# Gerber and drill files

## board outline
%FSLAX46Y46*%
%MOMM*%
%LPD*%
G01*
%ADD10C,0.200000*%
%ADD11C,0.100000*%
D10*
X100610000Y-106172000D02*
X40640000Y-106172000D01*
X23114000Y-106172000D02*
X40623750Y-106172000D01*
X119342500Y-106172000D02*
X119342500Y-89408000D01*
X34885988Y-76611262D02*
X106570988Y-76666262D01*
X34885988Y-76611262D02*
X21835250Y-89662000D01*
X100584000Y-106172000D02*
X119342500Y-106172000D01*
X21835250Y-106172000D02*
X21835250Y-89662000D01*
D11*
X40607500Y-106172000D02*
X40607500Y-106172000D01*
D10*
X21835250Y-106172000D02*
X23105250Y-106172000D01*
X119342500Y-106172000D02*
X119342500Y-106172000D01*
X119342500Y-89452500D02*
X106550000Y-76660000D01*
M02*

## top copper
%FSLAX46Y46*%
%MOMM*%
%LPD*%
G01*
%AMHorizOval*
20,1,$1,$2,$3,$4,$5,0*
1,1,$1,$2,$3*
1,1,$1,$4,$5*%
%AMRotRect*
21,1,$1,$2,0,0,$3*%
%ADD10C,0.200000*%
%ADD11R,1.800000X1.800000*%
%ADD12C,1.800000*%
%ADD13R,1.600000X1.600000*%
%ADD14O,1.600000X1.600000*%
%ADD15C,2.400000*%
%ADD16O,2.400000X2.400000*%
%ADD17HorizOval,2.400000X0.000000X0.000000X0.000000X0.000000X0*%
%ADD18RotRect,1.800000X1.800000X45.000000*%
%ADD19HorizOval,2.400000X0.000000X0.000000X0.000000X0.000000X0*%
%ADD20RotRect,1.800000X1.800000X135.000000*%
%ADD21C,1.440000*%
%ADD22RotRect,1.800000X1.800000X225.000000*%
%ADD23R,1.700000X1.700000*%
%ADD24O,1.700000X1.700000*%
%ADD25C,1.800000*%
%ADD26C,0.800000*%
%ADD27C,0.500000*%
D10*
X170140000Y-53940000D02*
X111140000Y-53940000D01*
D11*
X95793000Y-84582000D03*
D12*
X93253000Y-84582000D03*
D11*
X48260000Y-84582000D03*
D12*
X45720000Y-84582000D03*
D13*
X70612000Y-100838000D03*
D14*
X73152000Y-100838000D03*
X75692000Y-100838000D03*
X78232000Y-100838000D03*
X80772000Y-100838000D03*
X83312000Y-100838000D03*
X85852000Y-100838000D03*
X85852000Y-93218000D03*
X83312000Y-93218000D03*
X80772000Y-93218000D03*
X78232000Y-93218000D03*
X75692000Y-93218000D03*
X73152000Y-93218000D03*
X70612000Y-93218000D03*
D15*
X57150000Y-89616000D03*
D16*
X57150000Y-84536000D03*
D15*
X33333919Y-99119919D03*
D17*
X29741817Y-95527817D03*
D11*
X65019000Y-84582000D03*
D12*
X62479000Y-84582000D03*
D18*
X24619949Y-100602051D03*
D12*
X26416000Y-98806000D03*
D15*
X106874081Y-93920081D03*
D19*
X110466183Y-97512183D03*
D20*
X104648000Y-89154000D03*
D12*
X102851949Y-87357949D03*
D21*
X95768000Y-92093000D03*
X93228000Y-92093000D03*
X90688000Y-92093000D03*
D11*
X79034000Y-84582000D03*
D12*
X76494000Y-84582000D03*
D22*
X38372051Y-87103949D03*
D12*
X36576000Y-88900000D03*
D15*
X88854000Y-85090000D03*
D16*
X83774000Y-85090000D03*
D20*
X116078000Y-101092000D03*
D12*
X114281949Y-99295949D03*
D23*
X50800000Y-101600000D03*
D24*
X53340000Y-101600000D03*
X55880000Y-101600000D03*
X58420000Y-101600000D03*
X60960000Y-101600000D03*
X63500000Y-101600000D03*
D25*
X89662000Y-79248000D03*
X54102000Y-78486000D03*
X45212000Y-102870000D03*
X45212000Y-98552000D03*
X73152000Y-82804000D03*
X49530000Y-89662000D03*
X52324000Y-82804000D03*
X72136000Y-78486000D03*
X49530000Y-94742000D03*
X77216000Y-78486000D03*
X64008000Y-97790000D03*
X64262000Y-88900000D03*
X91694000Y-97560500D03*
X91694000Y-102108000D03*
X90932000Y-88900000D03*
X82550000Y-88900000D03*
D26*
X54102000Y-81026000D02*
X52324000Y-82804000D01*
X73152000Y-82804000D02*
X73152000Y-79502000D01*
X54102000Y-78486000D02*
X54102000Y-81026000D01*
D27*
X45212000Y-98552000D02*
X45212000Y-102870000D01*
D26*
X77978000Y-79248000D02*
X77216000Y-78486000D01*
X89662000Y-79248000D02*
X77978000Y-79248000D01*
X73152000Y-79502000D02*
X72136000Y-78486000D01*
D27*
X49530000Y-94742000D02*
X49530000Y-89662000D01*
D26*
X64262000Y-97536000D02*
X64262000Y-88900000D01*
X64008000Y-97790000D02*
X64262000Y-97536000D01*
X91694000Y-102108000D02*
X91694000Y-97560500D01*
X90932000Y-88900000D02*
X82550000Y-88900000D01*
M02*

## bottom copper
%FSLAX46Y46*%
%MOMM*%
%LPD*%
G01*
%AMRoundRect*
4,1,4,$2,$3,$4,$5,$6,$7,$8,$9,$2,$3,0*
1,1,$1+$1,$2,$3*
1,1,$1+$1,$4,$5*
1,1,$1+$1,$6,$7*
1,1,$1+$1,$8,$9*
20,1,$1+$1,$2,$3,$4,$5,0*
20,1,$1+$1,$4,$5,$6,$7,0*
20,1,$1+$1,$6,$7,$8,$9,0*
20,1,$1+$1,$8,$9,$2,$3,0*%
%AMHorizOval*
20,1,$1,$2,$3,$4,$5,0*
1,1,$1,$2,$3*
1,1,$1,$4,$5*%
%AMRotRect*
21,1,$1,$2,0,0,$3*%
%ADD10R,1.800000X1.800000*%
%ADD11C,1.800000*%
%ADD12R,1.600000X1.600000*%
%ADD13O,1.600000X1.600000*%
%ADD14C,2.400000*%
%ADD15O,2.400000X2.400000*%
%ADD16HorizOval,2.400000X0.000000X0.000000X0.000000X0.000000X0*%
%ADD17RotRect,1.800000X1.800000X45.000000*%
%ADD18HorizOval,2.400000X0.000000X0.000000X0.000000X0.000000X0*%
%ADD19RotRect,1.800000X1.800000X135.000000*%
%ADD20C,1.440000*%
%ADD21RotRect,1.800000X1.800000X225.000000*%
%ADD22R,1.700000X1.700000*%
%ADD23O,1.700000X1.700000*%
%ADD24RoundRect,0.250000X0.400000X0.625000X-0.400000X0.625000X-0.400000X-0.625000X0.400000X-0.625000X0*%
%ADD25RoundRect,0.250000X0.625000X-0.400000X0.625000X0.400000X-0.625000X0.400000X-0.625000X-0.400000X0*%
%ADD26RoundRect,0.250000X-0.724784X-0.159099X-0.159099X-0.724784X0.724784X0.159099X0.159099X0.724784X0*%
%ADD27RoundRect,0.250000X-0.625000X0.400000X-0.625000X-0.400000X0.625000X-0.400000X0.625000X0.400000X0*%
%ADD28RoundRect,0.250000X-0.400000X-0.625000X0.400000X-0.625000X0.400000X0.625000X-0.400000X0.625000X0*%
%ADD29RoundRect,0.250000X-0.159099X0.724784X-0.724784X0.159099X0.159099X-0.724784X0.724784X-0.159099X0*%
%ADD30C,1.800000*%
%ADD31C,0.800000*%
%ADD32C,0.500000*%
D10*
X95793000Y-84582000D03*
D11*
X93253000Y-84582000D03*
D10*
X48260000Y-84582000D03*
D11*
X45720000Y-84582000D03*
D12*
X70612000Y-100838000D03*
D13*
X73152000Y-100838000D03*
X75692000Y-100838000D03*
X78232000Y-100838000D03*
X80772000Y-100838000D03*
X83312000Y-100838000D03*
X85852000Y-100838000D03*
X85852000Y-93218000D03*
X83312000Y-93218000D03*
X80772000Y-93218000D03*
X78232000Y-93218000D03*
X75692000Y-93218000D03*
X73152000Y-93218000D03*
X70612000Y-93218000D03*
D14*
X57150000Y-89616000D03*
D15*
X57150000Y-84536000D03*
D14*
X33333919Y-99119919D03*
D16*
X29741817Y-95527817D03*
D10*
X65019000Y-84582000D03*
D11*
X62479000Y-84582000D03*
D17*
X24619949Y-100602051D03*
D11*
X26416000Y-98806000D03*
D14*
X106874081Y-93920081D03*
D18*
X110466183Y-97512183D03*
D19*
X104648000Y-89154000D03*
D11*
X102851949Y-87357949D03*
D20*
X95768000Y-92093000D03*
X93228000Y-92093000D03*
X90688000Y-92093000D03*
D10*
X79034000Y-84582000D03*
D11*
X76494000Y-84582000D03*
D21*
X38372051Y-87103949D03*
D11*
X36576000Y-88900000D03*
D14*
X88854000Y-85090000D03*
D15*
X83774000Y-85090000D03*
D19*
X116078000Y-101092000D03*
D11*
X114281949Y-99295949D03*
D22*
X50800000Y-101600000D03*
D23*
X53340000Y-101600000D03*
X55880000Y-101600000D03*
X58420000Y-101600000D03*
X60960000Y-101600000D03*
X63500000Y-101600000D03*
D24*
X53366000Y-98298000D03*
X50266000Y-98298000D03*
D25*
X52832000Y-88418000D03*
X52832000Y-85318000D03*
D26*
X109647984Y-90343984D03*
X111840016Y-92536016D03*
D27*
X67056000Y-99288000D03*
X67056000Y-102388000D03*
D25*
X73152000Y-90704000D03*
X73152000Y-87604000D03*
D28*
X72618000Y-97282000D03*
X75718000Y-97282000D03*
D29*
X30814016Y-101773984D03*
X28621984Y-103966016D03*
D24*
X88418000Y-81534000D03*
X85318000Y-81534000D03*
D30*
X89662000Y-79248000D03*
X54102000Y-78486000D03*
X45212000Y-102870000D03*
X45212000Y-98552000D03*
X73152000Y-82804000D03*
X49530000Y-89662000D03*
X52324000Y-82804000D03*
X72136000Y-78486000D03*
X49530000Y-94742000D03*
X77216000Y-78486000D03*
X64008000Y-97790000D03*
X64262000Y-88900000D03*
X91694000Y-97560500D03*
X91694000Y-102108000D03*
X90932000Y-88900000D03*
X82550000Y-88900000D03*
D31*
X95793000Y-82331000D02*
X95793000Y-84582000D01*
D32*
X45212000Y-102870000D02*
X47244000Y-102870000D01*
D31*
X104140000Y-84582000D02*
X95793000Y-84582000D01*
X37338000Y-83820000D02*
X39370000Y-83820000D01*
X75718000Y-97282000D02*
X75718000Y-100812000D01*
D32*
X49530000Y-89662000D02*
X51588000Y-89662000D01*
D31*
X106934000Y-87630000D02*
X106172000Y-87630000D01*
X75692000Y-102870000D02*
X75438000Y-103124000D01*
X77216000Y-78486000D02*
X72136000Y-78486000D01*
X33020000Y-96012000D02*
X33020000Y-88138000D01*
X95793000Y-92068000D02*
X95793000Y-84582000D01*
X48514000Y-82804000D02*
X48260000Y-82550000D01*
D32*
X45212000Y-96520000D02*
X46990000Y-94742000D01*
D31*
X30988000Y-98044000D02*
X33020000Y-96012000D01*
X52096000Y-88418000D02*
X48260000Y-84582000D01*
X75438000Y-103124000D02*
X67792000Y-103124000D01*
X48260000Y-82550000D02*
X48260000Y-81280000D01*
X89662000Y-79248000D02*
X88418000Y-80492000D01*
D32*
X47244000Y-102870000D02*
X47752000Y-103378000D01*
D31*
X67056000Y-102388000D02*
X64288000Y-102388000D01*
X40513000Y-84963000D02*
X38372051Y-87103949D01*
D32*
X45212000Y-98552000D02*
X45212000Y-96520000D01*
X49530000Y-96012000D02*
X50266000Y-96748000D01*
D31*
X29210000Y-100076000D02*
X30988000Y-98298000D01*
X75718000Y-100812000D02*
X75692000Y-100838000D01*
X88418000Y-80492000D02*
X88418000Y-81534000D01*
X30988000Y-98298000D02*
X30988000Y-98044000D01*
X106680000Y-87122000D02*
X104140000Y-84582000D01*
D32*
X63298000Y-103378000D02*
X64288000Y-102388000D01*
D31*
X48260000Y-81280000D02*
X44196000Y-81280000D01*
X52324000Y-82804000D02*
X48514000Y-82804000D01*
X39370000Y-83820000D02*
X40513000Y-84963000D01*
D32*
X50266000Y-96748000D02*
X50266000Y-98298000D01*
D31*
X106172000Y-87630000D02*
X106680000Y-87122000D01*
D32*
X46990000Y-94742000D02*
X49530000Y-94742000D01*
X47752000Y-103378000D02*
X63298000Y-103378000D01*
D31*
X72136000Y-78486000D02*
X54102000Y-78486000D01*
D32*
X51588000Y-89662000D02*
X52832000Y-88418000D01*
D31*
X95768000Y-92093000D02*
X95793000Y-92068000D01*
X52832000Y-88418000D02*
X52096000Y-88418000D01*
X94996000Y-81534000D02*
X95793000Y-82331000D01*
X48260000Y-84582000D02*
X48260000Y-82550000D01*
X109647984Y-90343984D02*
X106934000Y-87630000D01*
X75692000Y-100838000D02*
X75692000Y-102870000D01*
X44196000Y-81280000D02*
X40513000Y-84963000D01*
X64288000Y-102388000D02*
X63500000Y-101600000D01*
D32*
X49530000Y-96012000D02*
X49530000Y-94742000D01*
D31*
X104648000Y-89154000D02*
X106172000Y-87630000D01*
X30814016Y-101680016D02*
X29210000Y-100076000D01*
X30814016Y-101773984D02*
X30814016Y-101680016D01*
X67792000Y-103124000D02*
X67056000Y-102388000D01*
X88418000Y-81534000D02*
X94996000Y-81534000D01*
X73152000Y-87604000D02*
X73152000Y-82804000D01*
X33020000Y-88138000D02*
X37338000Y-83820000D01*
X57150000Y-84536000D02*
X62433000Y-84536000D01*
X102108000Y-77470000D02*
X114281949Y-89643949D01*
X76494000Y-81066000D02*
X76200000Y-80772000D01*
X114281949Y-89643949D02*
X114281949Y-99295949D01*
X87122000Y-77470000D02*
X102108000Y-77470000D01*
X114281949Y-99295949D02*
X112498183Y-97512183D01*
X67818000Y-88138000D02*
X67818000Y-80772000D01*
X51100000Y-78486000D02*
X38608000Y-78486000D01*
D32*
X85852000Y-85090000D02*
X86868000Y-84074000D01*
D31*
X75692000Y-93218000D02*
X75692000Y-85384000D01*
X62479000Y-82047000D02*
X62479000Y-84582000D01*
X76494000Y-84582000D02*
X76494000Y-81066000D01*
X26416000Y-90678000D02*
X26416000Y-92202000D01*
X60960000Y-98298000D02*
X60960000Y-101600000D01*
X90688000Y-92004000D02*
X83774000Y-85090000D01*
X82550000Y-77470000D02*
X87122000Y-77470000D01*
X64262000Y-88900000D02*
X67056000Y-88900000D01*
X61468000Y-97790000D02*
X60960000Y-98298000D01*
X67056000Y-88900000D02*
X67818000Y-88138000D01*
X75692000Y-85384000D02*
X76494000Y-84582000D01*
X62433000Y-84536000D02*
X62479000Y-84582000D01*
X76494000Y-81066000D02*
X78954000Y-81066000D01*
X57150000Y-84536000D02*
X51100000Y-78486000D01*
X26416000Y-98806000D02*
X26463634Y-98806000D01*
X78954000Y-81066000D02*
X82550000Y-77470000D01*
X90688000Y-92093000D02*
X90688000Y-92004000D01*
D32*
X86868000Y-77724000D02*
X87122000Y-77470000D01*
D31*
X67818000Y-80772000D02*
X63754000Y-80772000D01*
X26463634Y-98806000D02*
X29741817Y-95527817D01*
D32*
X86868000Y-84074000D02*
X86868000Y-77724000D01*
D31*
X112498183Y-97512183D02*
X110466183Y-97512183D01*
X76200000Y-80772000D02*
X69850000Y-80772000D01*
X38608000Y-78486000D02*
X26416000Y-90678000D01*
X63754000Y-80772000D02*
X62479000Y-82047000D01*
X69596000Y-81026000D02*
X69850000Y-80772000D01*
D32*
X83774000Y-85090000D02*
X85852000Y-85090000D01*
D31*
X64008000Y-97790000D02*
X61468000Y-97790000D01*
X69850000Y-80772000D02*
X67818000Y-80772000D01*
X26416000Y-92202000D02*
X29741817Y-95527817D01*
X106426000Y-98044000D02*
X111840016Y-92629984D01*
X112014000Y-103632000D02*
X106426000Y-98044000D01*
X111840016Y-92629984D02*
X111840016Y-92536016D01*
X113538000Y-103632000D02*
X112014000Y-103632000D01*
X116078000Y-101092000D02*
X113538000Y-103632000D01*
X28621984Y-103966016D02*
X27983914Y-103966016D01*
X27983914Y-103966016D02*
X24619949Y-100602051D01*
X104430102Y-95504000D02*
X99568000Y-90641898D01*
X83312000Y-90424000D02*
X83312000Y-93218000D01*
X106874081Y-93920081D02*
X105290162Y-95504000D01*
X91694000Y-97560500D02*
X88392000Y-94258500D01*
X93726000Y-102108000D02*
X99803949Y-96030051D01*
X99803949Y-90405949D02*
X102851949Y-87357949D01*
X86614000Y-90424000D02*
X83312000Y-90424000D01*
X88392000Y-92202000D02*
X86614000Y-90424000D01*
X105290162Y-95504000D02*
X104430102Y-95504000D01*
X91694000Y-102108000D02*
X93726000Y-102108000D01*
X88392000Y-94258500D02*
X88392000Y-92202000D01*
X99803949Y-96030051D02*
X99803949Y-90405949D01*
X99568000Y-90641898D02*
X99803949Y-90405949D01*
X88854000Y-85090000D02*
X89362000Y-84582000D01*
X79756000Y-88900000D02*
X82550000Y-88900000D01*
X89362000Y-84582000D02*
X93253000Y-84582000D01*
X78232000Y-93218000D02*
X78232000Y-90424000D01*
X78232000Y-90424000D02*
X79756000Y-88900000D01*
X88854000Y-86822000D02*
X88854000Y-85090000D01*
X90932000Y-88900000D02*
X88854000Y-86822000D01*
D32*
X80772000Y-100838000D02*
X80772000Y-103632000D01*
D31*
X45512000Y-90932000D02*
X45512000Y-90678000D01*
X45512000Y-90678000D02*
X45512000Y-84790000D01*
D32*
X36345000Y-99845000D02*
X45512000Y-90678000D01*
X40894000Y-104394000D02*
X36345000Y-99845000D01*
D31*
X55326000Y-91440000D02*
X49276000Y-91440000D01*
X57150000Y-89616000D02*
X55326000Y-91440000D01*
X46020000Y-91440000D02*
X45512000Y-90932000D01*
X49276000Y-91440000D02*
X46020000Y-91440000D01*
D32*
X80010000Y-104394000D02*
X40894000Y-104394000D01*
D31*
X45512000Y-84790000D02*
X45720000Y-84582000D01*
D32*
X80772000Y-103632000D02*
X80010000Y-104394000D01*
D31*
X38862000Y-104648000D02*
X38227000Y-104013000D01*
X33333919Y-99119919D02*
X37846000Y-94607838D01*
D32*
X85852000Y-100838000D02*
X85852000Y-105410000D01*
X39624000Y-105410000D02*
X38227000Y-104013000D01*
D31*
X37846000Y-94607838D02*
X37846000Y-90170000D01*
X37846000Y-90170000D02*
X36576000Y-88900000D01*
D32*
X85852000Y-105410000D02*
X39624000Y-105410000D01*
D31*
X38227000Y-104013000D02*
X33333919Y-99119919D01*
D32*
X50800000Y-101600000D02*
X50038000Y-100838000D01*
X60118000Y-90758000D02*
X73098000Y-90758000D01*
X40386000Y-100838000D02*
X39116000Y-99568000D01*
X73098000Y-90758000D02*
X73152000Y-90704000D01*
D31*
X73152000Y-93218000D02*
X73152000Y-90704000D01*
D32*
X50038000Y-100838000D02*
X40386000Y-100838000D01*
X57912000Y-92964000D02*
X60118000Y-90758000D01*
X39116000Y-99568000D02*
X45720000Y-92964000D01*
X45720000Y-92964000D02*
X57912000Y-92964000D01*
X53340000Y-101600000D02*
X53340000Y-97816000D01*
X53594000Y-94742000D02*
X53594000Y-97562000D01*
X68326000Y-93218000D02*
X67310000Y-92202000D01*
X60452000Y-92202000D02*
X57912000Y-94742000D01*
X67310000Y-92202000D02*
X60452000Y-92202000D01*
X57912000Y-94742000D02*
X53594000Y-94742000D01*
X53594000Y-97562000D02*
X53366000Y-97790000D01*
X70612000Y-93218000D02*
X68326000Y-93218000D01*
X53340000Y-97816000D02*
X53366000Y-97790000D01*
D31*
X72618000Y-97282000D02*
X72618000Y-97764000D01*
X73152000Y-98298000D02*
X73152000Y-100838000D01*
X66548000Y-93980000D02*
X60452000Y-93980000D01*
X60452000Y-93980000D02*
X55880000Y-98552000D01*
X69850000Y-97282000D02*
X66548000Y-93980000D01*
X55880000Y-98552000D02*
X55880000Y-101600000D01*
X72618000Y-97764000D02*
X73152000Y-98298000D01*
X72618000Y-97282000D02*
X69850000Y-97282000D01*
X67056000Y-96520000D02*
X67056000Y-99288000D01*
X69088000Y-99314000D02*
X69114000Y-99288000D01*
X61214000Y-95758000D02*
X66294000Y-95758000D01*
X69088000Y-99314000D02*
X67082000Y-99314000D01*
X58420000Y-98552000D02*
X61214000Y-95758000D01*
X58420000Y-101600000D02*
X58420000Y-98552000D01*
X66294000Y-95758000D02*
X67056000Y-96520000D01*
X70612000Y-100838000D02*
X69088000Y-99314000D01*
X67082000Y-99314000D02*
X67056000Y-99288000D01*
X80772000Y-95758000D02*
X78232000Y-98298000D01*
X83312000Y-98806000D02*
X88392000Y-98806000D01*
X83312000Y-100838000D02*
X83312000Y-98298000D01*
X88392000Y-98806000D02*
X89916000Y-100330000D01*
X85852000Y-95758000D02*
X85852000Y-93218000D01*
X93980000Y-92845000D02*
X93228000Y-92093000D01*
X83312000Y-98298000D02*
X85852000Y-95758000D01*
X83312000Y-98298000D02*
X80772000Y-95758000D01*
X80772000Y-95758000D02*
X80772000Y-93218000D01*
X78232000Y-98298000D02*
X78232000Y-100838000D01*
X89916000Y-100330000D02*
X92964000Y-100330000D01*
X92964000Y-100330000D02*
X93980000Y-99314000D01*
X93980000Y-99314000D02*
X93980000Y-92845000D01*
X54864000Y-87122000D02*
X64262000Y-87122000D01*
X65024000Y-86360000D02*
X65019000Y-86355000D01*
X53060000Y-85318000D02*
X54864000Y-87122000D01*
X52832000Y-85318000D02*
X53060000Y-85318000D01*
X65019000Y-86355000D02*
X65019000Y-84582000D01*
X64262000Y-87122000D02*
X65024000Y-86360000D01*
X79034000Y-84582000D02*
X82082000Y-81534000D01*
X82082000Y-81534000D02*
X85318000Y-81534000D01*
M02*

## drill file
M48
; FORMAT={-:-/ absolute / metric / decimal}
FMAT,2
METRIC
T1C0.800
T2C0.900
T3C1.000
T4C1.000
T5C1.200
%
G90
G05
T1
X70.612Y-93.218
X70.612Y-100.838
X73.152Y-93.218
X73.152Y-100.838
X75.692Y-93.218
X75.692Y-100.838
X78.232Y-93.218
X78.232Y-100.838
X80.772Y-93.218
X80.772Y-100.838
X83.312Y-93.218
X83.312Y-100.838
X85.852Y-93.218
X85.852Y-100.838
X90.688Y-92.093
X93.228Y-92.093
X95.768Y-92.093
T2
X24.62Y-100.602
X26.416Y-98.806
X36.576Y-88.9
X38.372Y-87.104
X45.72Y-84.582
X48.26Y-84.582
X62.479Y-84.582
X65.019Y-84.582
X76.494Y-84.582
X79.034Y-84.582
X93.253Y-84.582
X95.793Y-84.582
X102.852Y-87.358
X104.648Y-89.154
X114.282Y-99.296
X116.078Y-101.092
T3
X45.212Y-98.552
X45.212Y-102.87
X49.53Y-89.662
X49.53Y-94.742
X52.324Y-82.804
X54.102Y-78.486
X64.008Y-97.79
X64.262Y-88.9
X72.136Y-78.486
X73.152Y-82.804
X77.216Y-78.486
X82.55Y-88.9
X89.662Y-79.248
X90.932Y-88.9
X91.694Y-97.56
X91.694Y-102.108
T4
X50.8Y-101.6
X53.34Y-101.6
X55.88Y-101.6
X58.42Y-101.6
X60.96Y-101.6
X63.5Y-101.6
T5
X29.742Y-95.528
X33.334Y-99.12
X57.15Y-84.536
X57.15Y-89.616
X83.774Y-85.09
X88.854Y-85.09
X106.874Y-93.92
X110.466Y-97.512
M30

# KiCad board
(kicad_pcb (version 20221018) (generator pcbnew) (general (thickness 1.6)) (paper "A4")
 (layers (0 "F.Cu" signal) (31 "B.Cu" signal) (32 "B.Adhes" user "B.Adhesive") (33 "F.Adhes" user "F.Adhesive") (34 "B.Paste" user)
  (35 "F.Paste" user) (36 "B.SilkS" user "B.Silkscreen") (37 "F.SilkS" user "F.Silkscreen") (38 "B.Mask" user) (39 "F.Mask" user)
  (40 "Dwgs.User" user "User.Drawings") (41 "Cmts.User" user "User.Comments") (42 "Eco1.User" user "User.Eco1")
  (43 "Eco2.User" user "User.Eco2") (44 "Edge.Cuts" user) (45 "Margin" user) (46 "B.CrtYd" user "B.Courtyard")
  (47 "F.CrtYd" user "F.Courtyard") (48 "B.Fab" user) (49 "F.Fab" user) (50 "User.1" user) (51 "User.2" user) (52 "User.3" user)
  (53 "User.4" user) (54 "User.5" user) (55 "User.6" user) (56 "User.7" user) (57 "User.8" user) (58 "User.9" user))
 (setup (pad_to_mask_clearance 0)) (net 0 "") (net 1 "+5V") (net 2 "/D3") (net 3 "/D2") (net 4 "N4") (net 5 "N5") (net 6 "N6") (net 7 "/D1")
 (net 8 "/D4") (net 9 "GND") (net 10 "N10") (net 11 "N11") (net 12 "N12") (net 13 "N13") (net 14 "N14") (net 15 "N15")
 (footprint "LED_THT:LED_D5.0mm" (layer "F.Cu") (at 95.793 84.582 180)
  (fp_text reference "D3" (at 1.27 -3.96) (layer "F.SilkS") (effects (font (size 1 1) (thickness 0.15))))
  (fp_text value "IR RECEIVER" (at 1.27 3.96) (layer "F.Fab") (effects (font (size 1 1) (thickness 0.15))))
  (pad "1" thru_hole rect (at 0 0 180) (size 1.8 1.8) (drill 0.9) (layers "*.Cu" "*.Mask") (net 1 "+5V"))
  (pad "2" thru_hole circle (at 2.54 0 180) (size 1.8 1.8) (drill 0.9) (layers "*.Cu" "*.Mask") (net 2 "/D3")))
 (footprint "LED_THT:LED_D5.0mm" (layer "F.Cu") (at 48.26 84.582 180)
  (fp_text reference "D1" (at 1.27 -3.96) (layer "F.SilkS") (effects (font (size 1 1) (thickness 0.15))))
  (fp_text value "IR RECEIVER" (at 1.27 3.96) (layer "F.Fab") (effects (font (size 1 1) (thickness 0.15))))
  (pad "1" thru_hole rect (at 0 0 180) (size 1.8 1.8) (drill 0.9) (layers "*.Cu" "*.Mask") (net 1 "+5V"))
  (pad "2" thru_hole circle (at 2.54 0 180) (size 1.8 1.8) (drill 0.9) (layers "*.Cu" "*.Mask") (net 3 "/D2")))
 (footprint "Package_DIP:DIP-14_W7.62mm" (layer "F.Cu") (at 70.612 100.838 90)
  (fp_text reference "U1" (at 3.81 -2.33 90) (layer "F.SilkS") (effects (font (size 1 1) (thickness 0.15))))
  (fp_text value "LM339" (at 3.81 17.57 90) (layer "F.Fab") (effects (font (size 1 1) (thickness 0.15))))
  (pad "1" thru_hole rect (at 0 0 90) (size 1.6 1.6) (drill 0.8) (layers "*.Cu" "*.Mask") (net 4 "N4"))
  (pad "2" thru_hole oval (at 0 2.54 90) (size 1.6 1.6) (drill 0.8) (layers "*.Cu" "*.Mask") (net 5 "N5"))
  (pad "3" thru_hole oval (at 0 5.08 90) (size 1.6 1.6) (drill 0.8) (layers "*.Cu" "*.Mask") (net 1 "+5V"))
  (pad "4" thru_hole oval (at 0 7.62 90) (size 1.6 1.6) (drill 0.8) (layers "*.Cu" "*.Mask") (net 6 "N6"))
  (pad "5" thru_hole oval (at 0 10.16 90) (size 1.6 1.6) (drill 0.8) (layers "*.Cu" "*.Mask") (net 3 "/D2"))
  (pad "6" thru_hole oval (at 0 12.7 90) (size 1.6 1.6) (drill 0.8) (layers "*.Cu" "*.Mask") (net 6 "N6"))
  (pad "7" thru_hole oval (at 0 15.24 90) (size 1.6 1.6) (drill 0.8) (layers "*.Cu" "*.Mask") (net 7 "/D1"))
  (pad "8" thru_hole oval (at 7.62 15.24 90) (size 1.6 1.6) (drill 0.8) (layers "*.Cu" "*.Mask") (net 6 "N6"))
  (pad "9" thru_hole oval (at 7.62 12.7 90) (size 1.6 1.6) (drill 0.8) (layers "*.Cu" "*.Mask") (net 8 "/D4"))
  (pad "10" thru_hole oval (at 7.62 10.16 90) (size 1.6 1.6) (drill 0.8) (layers "*.Cu" "*.Mask") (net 6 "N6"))
  (pad "11" thru_hole oval (at 7.62 7.62 90) (size 1.6 1.6) (drill 0.8) (layers "*.Cu" "*.Mask") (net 2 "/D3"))
  (pad "12" thru_hole oval (at 7.62 5.08 90) (size 1.6 1.6) (drill 0.8) (layers "*.Cu" "*.Mask") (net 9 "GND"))
  (pad "13" thru_hole oval (at 7.62 2.54 90) (size 1.6 1.6) (drill 0.8) (layers "*.Cu" "*.Mask") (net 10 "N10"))
  (pad "14" thru_hole oval (at 7.62 0 90) (size 1.6 1.6) (drill 0.8) (layers "*.Cu" "*.Mask") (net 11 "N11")))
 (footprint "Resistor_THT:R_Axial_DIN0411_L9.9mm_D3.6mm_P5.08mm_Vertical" (layer "F.Cu") (at 57.15 89.616 90)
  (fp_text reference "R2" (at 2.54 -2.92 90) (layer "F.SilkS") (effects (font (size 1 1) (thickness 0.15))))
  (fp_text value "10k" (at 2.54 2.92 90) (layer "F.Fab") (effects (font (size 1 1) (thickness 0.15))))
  (pad "1" thru_hole circle (at 0 0 90) (size 2.4 2.4) (drill 1.2) (layers "*.Cu" "*.Mask") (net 3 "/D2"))
  (pad "2" thru_hole oval (at 5.08 0 90) (size 2.4 2.4) (drill 1.2) (layers "*.Cu" "*.Mask") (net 9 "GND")))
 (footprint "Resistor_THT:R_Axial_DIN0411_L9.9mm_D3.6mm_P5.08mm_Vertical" (layer "F.Cu") (at 33.333919 99.119919 135)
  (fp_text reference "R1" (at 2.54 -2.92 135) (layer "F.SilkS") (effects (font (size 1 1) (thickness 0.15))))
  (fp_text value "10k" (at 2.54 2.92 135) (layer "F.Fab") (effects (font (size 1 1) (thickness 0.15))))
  (pad "1" thru_hole circle (at 0 0 135) (size 2.4 2.4) (drill 1.2) (layers "*.Cu" "*.Mask") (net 7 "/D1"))
  (pad "2" thru_hole oval (at 5.08 0 135) (size 2.4 2.4) (drill 1.2) (layers "*.Cu" "*.Mask") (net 9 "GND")))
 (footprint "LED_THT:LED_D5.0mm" (layer "F.Cu") (at 65.019 84.582 180)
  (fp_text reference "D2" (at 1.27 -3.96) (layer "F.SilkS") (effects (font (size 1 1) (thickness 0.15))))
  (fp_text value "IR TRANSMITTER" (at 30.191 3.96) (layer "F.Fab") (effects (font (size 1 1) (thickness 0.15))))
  (pad "1" thru_hole rect (at 0 0 180) (size 1.8 1.8) (drill 0.9) (layers "*.Cu" "*.Mask") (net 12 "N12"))
  (pad "2" thru_hole circle (at 2.54 0 180) (size 1.8 1.8) (drill 0.9) (layers "*.Cu" "*.Mask") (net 9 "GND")))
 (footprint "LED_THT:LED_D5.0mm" (layer "F.Cu") (at 24.619949 100.602051 45)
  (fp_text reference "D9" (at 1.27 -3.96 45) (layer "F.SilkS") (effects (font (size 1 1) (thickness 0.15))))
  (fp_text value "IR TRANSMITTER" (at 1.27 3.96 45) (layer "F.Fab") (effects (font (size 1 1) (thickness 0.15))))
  (pad "1" thru_hole rect (at 0 0 45) (size 1.8 1.8) (drill 0.9) (layers "*.Cu" "*.Mask") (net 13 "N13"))
  (pad "2" thru_hole circle (at 2.54 0 45) (size 1.8 1.8) (drill 0.9) (layers "*.Cu" "*.Mask") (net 9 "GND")))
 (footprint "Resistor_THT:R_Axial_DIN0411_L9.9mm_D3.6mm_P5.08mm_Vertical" (layer "F.Cu") (at 106.874081 93.920081 -45)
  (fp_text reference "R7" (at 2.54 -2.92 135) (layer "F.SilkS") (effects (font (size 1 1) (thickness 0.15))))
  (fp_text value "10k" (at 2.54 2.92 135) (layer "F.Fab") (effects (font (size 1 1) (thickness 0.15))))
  (pad "1" thru_hole circle (at 0 0 315) (size 2.4 2.4) (drill 1.2) (layers "*.Cu" "*.Mask") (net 8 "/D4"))
  (pad "2" thru_hole oval (at 5.08 0 315) (size 2.4 2.4) (drill 1.2) (layers "*.Cu" "*.Mask") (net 9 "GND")))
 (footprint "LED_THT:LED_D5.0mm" (layer "F.Cu") (at 104.648 89.154 135)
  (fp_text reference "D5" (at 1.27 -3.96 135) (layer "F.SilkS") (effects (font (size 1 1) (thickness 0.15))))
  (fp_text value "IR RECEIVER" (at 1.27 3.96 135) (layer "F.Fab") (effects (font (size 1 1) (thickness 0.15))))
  (pad "1" thru_hole rect (at 0 0 135) (size 1.8 1.8) (drill 0.9) (layers "*.Cu" "*.Mask") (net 1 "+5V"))
  (pad "2" thru_hole circle (at 2.54 0 135) (size 1.8 1.8) (drill 0.9) (layers "*.Cu" "*.Mask") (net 8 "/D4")))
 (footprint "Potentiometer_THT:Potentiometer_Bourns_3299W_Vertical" (layer "F.Cu") (at 95.768 92.093)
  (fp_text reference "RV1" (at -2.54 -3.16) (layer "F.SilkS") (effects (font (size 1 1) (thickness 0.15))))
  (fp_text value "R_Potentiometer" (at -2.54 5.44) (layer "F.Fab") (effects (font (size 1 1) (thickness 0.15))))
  (pad "1" thru_hole circle (at 0 0) (size 1.44 1.44) (drill 0.8) (layers "*.Cu" "*.Mask") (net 1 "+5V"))
  (pad "2" thru_hole circle (at -2.54 0) (size 1.44 1.44) (drill 0.8) (layers "*.Cu" "*.Mask") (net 6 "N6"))
  (pad "3" thru_hole circle (at -5.08 0) (size 1.44 1.44) (drill 0.8) (layers "*.Cu" "*.Mask") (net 9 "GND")))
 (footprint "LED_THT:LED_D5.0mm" (layer "F.Cu") (at 79.034 84.582 180)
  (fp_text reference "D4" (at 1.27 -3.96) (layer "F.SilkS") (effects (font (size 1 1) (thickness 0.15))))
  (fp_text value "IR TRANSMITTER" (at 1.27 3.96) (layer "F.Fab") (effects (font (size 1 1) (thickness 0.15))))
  (pad "1" thru_hole rect (at 0 0 180) (size 1.8 1.8) (drill 0.9) (layers "*.Cu" "*.Mask") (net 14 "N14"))
  (pad "2" thru_hole circle (at 2.54 0 180) (size 1.8 1.8) (drill 0.9) (layers "*.Cu" "*.Mask") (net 9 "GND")))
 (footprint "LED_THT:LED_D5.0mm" (layer "F.Cu") (at 38.372051 87.103949 -135)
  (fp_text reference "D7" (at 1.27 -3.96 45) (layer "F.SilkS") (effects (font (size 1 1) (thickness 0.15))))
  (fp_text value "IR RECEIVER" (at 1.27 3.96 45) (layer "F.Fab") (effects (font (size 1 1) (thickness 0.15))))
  (pad "1" thru_hole rect (at 0 0 225) (size 1.8 1.8) (drill 0.9) (layers "*.Cu" "*.Mask") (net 1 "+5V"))
  (pad "2" thru_hole circle (at 2.54 0 225) (size 1.8 1.8) (drill 0.9) (layers "*.Cu" "*.Mask") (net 7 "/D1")))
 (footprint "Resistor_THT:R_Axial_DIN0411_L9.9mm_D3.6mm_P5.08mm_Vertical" (layer "F.Cu") (at 88.854 85.09 180)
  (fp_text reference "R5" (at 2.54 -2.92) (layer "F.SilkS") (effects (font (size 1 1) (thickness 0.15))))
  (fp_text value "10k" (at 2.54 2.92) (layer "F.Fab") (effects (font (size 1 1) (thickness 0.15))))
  (pad "1" thru_hole circle (at 0 0 180) (size 2.4 2.4) (drill 1.2) (layers "*.Cu" "*.Mask") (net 2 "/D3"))
  (pad "2" thru_hole oval (at 5.08 0 180) (size 2.4 2.4) (drill 1.2) (layers "*.Cu" "*.Mask") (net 9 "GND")))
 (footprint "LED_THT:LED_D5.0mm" (layer "F.Cu") (at 116.078 101.092 135)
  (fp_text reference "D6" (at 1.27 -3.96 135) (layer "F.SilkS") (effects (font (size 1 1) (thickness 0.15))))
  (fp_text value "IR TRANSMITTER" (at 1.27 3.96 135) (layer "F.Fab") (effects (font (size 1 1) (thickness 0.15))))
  (pad "1" thru_hole rect (at 0 0 135) (size 1.8 1.8) (drill 0.9) (layers "*.Cu" "*.Mask") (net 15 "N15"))
  (pad "2" thru_hole circle (at 2.54 0 135) (size 1.8 1.8) (drill 0.9) (layers "*.Cu" "*.Mask") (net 9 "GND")))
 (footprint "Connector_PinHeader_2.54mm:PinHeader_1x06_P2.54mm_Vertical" (layer "F.Cu") (at 50.8 101.6 90)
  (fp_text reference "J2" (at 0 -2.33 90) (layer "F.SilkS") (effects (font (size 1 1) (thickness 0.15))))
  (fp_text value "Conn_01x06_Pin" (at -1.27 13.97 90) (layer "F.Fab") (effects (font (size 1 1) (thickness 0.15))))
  (pad "1" thru_hole rect (at 0 0 90) (size 1.7 1.7) (drill 1) (layers "*.Cu" "*.Mask") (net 10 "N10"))
  (pad "2" thru_hole oval (at 0 2.54 90) (size 1.7 1.7) (drill 1) (layers "*.Cu" "*.Mask") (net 11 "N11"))
  (pad "3" thru_hole oval (at 0 5.08 90) (size 1.7 1.7) (drill 1) (layers "*.Cu" "*.Mask") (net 5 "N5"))
  (pad "4" thru_hole oval (at 0 7.62 90) (size 1.7 1.7) (drill 1) (layers "*.Cu" "*.Mask") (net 4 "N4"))
  (pad "5" thru_hole oval (at 0 10.16 90) (size 1.7 1.7) (drill 1) (layers "*.Cu" "*.Mask") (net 9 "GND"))
  (pad "6" thru_hole oval (at 0 12.7 90) (size 1.7 1.7) (drill 1) (layers "*.Cu" "*.Mask") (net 1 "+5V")))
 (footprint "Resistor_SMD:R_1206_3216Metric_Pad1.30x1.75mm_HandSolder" (layer "B.Cu") (at 51.816 98.298 180)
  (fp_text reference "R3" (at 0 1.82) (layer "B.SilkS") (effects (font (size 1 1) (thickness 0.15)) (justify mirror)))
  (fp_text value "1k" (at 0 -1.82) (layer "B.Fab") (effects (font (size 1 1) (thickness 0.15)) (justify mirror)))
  (pad "1" smd roundrect (at -1.55 0 180) (size 1.3 1.75) (layers "B.Cu" "B.Paste" "B.Mask") (roundrect_rratio 0.192308) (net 11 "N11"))
  (pad "2" smd roundrect (at 1.55 0 180) (size 1.3 1.75) (layers "B.Cu" "B.Paste" "B.Mask") (roundrect_rratio 0.192308) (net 1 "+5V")))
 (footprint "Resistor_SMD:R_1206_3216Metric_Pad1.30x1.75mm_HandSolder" (layer "B.Cu") (at 52.832 86.868 90)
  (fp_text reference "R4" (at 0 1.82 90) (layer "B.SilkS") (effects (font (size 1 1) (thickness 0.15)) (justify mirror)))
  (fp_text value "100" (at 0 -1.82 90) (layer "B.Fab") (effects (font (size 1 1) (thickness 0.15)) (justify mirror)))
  (pad "1" smd roundrect (at -1.55 0 90) (size 1.3 1.75) (layers "B.Cu" "B.Paste" "B.Mask") (roundrect_rratio 0.192308) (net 1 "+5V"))
  (pad "2" smd roundrect (at 1.55 0 90) (size 1.3 1.75) (layers "B.Cu" "B.Paste" "B.Mask") (roundrect_rratio 0.192308) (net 12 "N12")))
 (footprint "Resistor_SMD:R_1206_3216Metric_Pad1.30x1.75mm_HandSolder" (layer "B.Cu") (at 110.744 91.44 -45)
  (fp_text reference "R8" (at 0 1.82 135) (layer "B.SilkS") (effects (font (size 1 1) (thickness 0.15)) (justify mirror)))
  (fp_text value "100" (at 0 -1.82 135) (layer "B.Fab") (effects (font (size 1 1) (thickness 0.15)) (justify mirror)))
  (pad "1" smd roundrect (at -1.55 0 315) (size 1.3 1.75) (layers "B.Cu" "B.Paste" "B.Mask") (roundrect_rratio 0.192308) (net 1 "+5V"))
  (pad "2" smd roundrect (at 1.55 0 315) (size 1.3 1.75) (layers "B.Cu" "B.Paste" "B.Mask") (roundrect_rratio 0.192308) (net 15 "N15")))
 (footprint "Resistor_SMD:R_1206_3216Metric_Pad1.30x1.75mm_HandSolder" (layer "B.Cu") (at 67.056 100.838 -90)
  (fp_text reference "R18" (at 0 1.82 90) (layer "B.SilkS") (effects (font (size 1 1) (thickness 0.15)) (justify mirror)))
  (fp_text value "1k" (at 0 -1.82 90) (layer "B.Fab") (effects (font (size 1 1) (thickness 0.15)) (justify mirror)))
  (pad "1" smd roundrect (at -1.55 0 270) (size 1.3 1.75) (layers "B.Cu" "B.Paste" "B.Mask") (roundrect_rratio 0.192308) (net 4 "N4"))
  (pad "2" smd roundrect (at 1.55 0 270) (size 1.3 1.75) (layers "B.Cu" "B.Paste" "B.Mask") (roundrect_rratio 0.192308) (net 1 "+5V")))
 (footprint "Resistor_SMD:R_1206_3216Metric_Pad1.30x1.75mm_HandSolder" (layer "B.Cu") (at 73.152 89.154 90)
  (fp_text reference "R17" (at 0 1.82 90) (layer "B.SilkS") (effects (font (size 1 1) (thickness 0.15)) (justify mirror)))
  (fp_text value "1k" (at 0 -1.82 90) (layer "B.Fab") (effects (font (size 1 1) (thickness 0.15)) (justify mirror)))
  (pad "1" smd roundrect (at -1.55 0 90) (size 1.3 1.75) (layers "B.Cu" "B.Paste" "B.Mask") (roundrect_rratio 0.192308) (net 10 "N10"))
  (pad "2" smd roundrect (at 1.55 0 90) (size 1.3 1.75) (layers "B.Cu" "B.Paste" "B.Mask") (roundrect_rratio 0.192308) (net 1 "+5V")))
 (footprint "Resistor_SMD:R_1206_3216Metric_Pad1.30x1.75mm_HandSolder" (layer "B.Cu") (at 74.168 97.282)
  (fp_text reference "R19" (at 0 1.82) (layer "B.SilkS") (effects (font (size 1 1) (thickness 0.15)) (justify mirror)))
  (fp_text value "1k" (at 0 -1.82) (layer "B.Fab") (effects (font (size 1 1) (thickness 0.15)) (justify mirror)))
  (pad "1" smd roundrect (at -1.55 0) (size 1.3 1.75) (layers "B.Cu" "B.Paste" "B.Mask") (roundrect_rratio 0.192308) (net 5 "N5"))
  (pad "2" smd roundrect (at 1.55 0) (size 1.3 1.75) (layers "B.Cu" "B.Paste" "B.Mask") (roundrect_rratio 0.192308) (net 1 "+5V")))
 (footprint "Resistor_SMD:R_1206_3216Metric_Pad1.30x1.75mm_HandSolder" (layer "B.Cu") (at 29.718 102.87 -135)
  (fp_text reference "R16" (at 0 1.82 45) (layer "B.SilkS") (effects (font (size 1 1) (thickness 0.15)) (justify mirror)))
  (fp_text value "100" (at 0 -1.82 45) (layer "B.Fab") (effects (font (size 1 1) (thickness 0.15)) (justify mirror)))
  (pad "1" smd roundrect (at -1.55 0 225) (size 1.3 1.75) (layers "B.Cu" "B.Paste" "B.Mask") (roundrect_rratio 0.192308) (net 1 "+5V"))
  (pad "2" smd roundrect (at 1.55 0 225) (size 1.3 1.75) (layers "B.Cu" "B.Paste" "B.Mask") (roundrect_rratio 0.192308) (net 13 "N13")))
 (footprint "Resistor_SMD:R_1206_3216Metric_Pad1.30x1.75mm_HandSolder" (layer "B.Cu") (at 86.868 81.534 180)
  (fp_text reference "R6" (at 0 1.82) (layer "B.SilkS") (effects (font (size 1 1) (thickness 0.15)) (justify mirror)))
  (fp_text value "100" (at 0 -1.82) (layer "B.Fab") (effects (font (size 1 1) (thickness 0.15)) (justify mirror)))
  (pad "1" smd roundrect (at -1.55 0 180) (size 1.3 1.75) (layers "B.Cu" "B.Paste" "B.Mask") (roundrect_rratio 0.192308) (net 1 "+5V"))
  (pad "2" smd roundrect (at 1.55 0 180) (size 1.3 1.75) (layers "B.Cu" "B.Paste" "B.Mask") (roundrect_rratio 0.192308) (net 14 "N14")))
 (gr_line locked (start 170.14 53.94) (end 111.14 53.94) (stroke (width 0.2) (type default)) (layer "F.Cu"))
 (gr_line (start 100.61 106.172) (end 40.64 106.172) (stroke (width 0.2) (type default)) (layer "Edge.Cuts"))
 (gr_line (start 23.114 106.172) (end 40.62375 106.172) (stroke (width 0.2) (type default)) (layer "Edge.Cuts"))
 (gr_line (start 119.3425 106.172) (end 119.3425 89.408) (stroke (width 0.2) (type default)) (layer "Edge.Cuts"))
 (gr_line (start 34.885988 76.611262) (end 106.570988 76.666262) (stroke (width 0.2) (type default)) (layer "Edge.Cuts"))
 (gr_line (start 34.885988 76.611262) (end 21.83525 89.662) (stroke (width 0.2) (type default)) (layer "Edge.Cuts"))
 (gr_line (start 100.584 106.172) (end 119.3425 106.172) (stroke (width 0.2) (type default)) (layer "Edge.Cuts"))
 (gr_line (start 21.83525 106.172) (end 21.83525 89.662) (stroke (width 0.2) (type default)) (layer "Edge.Cuts"))
 (gr_line (start 40.6075 106.172) (end 40.6075 106.172) (stroke (width 0.1) (type default)) (layer "Edge.Cuts"))
 (gr_line (start 21.83525 106.172) (end 23.10525 106.172) (stroke (width 0.2) (type default)) (layer "Edge.Cuts"))
 (gr_line (start 119.3425 106.172) (end 119.3425 106.172) (stroke (width 0.2) (type default)) (layer "Edge.Cuts"))
 (gr_line (start 119.3425 89.4525) (end 106.55 76.66) (stroke (width 0.2) (type default)) (layer "Edge.Cuts"))
 (segment (start 54.102 81.026) (end 52.324 82.804) (width 0.8) (layer "F.Cu") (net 1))
 (segment (start 73.152 82.804) (end 73.152 79.502) (width 0.8) (layer "F.Cu") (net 1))
 (segment (start 54.102 78.486) (end 54.102 81.026) (width 0.8) (layer "F.Cu") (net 1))
 (segment (start 45.212 98.552) (end 45.212 102.87) (width 0.5) (layer "F.Cu") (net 1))
 (segment (start 77.978 79.248) (end 77.216 78.486) (width 0.8) (layer "F.Cu") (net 1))
 (segment (start 89.662 79.248) (end 77.978 79.248) (width 0.8) (layer "F.Cu") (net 1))
 (segment (start 73.152 79.502) (end 72.136 78.486) (width 0.8) (layer "F.Cu") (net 1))
 (segment (start 49.53 94.742) (end 49.53 89.662) (width 0.5) (layer "F.Cu") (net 1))
 (via (at 89.662 79.248) (size 1.8) (drill 1) (layers "F.Cu" "B.Cu") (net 1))
 (via (at 54.102 78.486) (size 1.8) (drill 1) (layers "F.Cu" "B.Cu") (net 1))
 (via (at 45.212 102.87) (size 1.8) (drill 1) (layers "F.Cu" "B.Cu") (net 1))
 (via (at 45.212 98.552) (size 1.8) (drill 1) (layers "F.Cu" "B.Cu") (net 1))
 (via (at 73.152 82.804) (size 1.8) (drill 1) (layers "F.Cu" "B.Cu") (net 1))
 (via (at 49.53 89.662) (size 1.8) (drill 1) (layers "F.Cu" "B.Cu") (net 1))
 (via (at 52.324 82.804) (size 1.8) (drill 1) (layers "F.Cu" "B.Cu") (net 1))
 (via (at 72.136 78.486) (size 1.8) (drill 1) (layers "F.Cu" "B.Cu") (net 1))
 (via (at 49.53 94.742) (size 1.8) (drill 1) (layers "F.Cu" "B.Cu") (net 1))
 (via (at 77.216 78.486) (size 1.8) (drill 1) (layers "F.Cu" "B.Cu") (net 1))
 (segment (start 95.793 82.331) (end 95.793 84.582) (width 0.8) (layer "B.Cu") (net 1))
 (segment (start 45.212 102.87) (end 47.244 102.87) (width 0.5) (layer "B.Cu") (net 1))
 (segment (start 104.14 84.582) (end 95.793 84.582) (width 0.8) (layer "B.Cu") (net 1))
 (segment (start 37.338 83.82) (end 39.37 83.82) (width 0.8) (layer "B.Cu") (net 1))
 (segment (start 75.718 97.282) (end 75.718 100.812) (width 0.8) (layer "B.Cu") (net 1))
 (segment (start 49.53 89.662) (end 51.588 89.662) (width 0.5) (layer "B.Cu") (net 1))
 (segment (start 106.934 87.63) (end 106.172 87.63) (width 0.8) (layer "B.Cu") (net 1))
 (segment (start 75.692 102.87) (end 75.438 103.124) (width 0.8) (layer "B.Cu") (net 1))
 (segment (start 77.216 78.486) (end 72.136 78.486) (width 0.8) (layer "B.Cu") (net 1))
 (segment (start 33.02 96.012) (end 33.02 88.138) (width 0.8) (layer "B.Cu") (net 1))
 (segment (start 95.793 92.068) (end 95.793 84.582) (width 0.8) (layer "B.Cu") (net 1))
 (segment (start 48.514 82.804) (end 48.26 82.55) (width 0.8) (layer "B.Cu") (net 1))
 (segment (start 45.212 96.52) (end 46.99 94.742) (width 0.5) (layer "B.Cu") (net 1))
 (segment (start 30.988 98.044) (end 33.02 96.012) (width 0.8) (layer "B.Cu") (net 1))
 (segment (start 52.096 88.418) (end 48.26 84.582) (width 0.8) (layer "B.Cu") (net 1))
 (segment (start 75.438 103.124) (end 67.792 103.124) (width 0.8) (layer "B.Cu") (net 1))
 (segment (start 48.26 82.55) (end 48.26 81.28) (width 0.8) (layer "B.Cu") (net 1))
 (segment (start 89.662 79.248) (end 88.418 80.492) (width 0.8) (layer "B.Cu") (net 1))
 (segment (start 47.244 102.87) (end 47.752 103.378) (width 0.5) (layer "B.Cu") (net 1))
 (segment (start 67.056 102.388) (end 64.288 102.388) (width 0.8) (layer "B.Cu") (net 1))
 (segment (start 40.513 84.963) (end 38.372051 87.103949) (width 0.8) (layer "B.Cu") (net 1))
 (segment (start 45.212 98.552) (end 45.212 96.52) (width 0.5) (layer "B.Cu") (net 1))
 (segment (start 49.53 96.012) (end 50.266 96.748) (width 0.5) (layer "B.Cu") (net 1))
 (segment (start 29.21 100.076) (end 30.988 98.298) (width 0.8) (layer "B.Cu") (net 1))
 (segment (start 75.718 100.812) (end 75.692 100.838) (width 0.8) (layer "B.Cu") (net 1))
 (segment (start 88.418 80.492) (end 88.418 81.534) (width 0.8) (layer "B.Cu") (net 1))
 (segment (start 30.988 98.298) (end 30.988 98.044) (width 0.8) (layer "B.Cu") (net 1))
 (segment (start 106.68 87.122) (end 104.14 84.582) (width 0.8) (layer "B.Cu") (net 1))
 (segment (start 63.298 103.378) (end 64.288 102.388) (width 0.5) (layer "B.Cu") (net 1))
 (segment (start 48.26 81.28) (end 44.196 81.28) (width 0.8) (layer "B.Cu") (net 1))
 (segment (start 52.324 82.804) (end 48.514 82.804) (width 0.8) (layer "B.Cu") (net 1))
 (segment (start 39.37 83.82) (end 40.513 84.963) (width 0.8) (layer "B.Cu") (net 1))
 (segment (start 50.266 96.748) (end 50.266 98.298) (width 0.5) (layer "B.Cu") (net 1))
 (segment (start 106.172 87.63) (end 106.68 87.122) (width 0.8) (layer "B.Cu") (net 1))
 (segment (start 46.99 94.742) (end 49.53 94.742) (width 0.5) (layer "B.Cu") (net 1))
 (segment (start 47.752 103.378) (end 63.298 103.378) (width 0.5) (layer "B.Cu") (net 1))
 (segment (start 72.136 78.486) (end 54.102 78.486) (width 0.8) (layer "B.Cu") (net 1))
 (segment (start 51.588 89.662) (end 52.832 88.418) (width 0.5) (layer "B.Cu") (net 1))
 (segment (start 95.768 92.093) (end 95.793 92.068) (width 0.8) (layer "B.Cu") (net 1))
 (segment (start 52.832 88.418) (end 52.096 88.418) (width 0.8) (layer "B.Cu") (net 1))
 (segment (start 94.996 81.534) (end 95.793 82.331) (width 0.8) (layer "B.Cu") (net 1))
 (segment (start 48.26 84.582) (end 48.26 82.55) (width 0.8) (layer "B.Cu") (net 1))
 (segment (start 109.647984 90.343984) (end 106.934 87.63) (width 0.8) (layer "B.Cu") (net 1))
 (segment (start 75.692 100.838) (end 75.692 102.87) (width 0.8) (layer "B.Cu") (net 1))
 (segment (start 44.196 81.28) (end 40.513 84.963) (width 0.8) (layer "B.Cu") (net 1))
 (segment (start 64.288 102.388) (end 63.5 101.6) (width 0.8) (layer "B.Cu") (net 1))
 (segment (start 49.53 96.012) (end 49.53 94.742) (width 0.5) (layer "B.Cu") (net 1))
 (segment (start 104.648 89.154) (end 106.172 87.63) (width 0.8) (layer "B.Cu") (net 1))
 (segment (start 30.814016 101.680016) (end 29.21 100.076) (width 0.8) (layer "B.Cu") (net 1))
 (segment (start 30.814016 101.773984) (end 30.814016 101.680016) (width 0.8) (layer "B.Cu") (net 1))
 (segment (start 67.792 103.124) (end 67.056 102.388) (width 0.8) (layer "B.Cu") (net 1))
 (segment (start 88.418 81.534) (end 94.996 81.534) (width 0.8) (layer "B.Cu") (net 1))
 (segment (start 73.152 87.604) (end 73.152 82.804) (width 0.8) (layer "B.Cu") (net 1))
 (segment (start 33.02 88.138) (end 37.338 83.82) (width 0.8) (layer "B.Cu") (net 1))
 (segment (start 64.262 97.536) (end 64.262 88.9) (width 0.8) (layer "F.Cu") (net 9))
 (segment (start 64.008 97.79) (end 64.262 97.536) (width 0.8) (layer "F.Cu") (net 9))
 (via (at 64.008 97.79) (size 1.8) (drill 1) (layers "F.Cu" "B.Cu") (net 9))
 (via (at 64.262 88.9) (size 1.8) (drill 1) (layers "F.Cu" "B.Cu") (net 9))
 (segment (start 57.15 84.536) (end 62.433 84.536) (width 0.8) (layer "B.Cu") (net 9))
 (segment (start 102.108 77.47) (end 114.281949 89.643949) (width 0.8) (layer "B.Cu") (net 9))
 (segment (start 76.494 81.066) (end 76.2 80.772) (width 0.8) (layer "B.Cu") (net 9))
 (segment (start 114.281949 89.643949) (end 114.281949 99.295949) (width 0.8) (layer "B.Cu") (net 9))
 (segment (start 87.122 77.47) (end 102.108 77.47) (width 0.8) (layer "B.Cu") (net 9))
 (segment (start 114.281949 99.295949) (end 112.498183 97.512183) (width 0.8) (layer "B.Cu") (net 9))
 (segment (start 67.818 88.138) (end 67.818 80.772) (width 0.8) (layer "B.Cu") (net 9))
 (segment (start 51.1 78.486) (end 38.608 78.486) (width 0.8) (layer "B.Cu") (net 9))
 (segment (start 85.852 85.09) (end 86.868 84.074) (width 0.5) (layer "B.Cu") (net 9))
 (segment (start 75.692 93.218) (end 75.692 85.384) (width 0.8) (layer "B.Cu") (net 9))
 (segment (start 62.479 82.047) (end 62.479 84.582) (width 0.8) (layer "B.Cu") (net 9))
 (segment (start 76.494 84.582) (end 76.494 81.066) (width 0.8) (layer "B.Cu") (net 9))
 (segment (start 26.416 90.678) (end 26.416 92.202) (width 0.8) (layer "B.Cu") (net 9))
 (segment (start 60.96 98.298) (end 60.96 101.6) (width 0.8) (layer "B.Cu") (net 9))
 (segment (start 90.688 92.004) (end 83.774 85.09) (width 0.8) (layer "B.Cu") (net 9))
 (segment (start 82.55 77.47) (end 87.122 77.47) (width 0.8) (layer "B.Cu") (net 9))
 (segment (start 64.262 88.9) (end 67.056 88.9) (width 0.8) (layer "B.Cu") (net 9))
 (segment (start 61.468 97.79) (end 60.96 98.298) (width 0.8) (layer "B.Cu") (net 9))
 (segment (start 67.056 88.9) (end 67.818 88.138) (width 0.8) (layer "B.Cu") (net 9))
 (segment (start 75.692 85.384) (end 76.494 84.582) (width 0.8) (layer "B.Cu") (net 9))
 (segment (start 62.433 84.536) (end 62.479 84.582) (width 0.8) (layer "B.Cu") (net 9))
 (segment (start 76.494 81.066) (end 78.954 81.066) (width 0.8) (layer "B.Cu") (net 9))
 (segment (start 57.15 84.536) (end 51.1 78.486) (width 0.8) (layer "B.Cu") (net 9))
 (segment (start 26.416 98.806) (end 26.463634 98.806) (width 0.8) (layer "B.Cu") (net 9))
 (segment (start 78.954 81.066) (end 82.55 77.47) (width 0.8) (layer "B.Cu") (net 9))
 (segment (start 90.688 92.093) (end 90.688 92.004) (width 0.8) (layer "B.Cu") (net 9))
 (segment (start 86.868 77.724) (end 87.122 77.47) (width 0.5) (layer "B.Cu") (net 9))
 (segment (start 67.818 80.772) (end 63.754 80.772) (width 0.8) (layer "B.Cu") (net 9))
 (segment (start 26.463634 98.806) (end 29.741817 95.527817) (width 0.8) (layer "B.Cu") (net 9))
 (segment (start 86.868 84.074) (end 86.868 77.724) (width 0.5) (layer "B.Cu") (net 9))
 (segment (start 112.498183 97.512183) (end 110.466183 97.512183) (width 0.8) (layer "B.Cu") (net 9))
 (segment (start 76.2 80.772) (end 69.85 80.772) (width 0.8) (layer "B.Cu") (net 9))
 (segment (start 38.608 78.486) (end 26.416 90.678) (width 0.8) (layer "B.Cu") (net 9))
 (segment (start 63.754 80.772) (end 62.479 82.047) (width 0.8) (layer "B.Cu") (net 9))
 (segment (start 69.596 81.026) (end 69.85 80.772) (width 0.8) (layer "B.Cu") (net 9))
 (segment (start 83.774 85.09) (end 85.852 85.09) (width 0.5) (layer "B.Cu") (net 9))
 (segment (start 64.008 97.79) (end 61.468 97.79) (width 0.8) (layer "B.Cu") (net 9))
 (segment (start 69.85 80.772) (end 67.818 80.772) (width 0.8) (layer "B.Cu") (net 9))
 (segment (start 26.416 92.202) (end 29.741817 95.527817) (width 0.8) (layer "B.Cu") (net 9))
 (segment (start 106.426 98.044) (end 111.840016 92.629984) (width 0.8) (layer "B.Cu") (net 15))
 (segment (start 112.014 103.632) (end 106.426 98.044) (width 0.8) (layer "B.Cu") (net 15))
 (segment (start 111.840016 92.629984) (end 111.840016 92.536016) (width 0.8) (layer "B.Cu") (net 15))
 (segment (start 113.538 103.632) (end 112.014 103.632) (width 0.8) (layer "B.Cu") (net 15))
 (segment (start 116.078 101.092) (end 113.538 103.632) (width 0.8) (layer "B.Cu") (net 15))
 (segment (start 28.621984 103.966016) (end 27.983914 103.966016) (width 0.8) (layer "B.Cu") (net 13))
 (segment (start 27.983914 103.966016) (end 24.619949 100.602051) (width 0.8) (layer "B.Cu") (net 13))
 (segment (start 91.694 102.108) (end 91.694 97.5605) (width 0.8) (layer "F.Cu") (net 8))
 (via (at 91.694 97.5605) (size 1.8) (drill 1) (layers "F.Cu" "B.Cu") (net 8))
 (via (at 91.694 102.108) (size 1.8) (drill 1) (layers "F.Cu" "B.Cu") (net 8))
 (segment (start 104.430102 95.504) (end 99.568 90.641898) (width 0.8) (layer "B.Cu") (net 8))
 (segment (start 83.312 90.424) (end 83.312 93.218) (width 0.8) (layer "B.Cu") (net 8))
 (segment (start 106.874081 93.920081) (end 105.290162 95.504) (width 0.8) (layer "B.Cu") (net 8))
 (segment (start 91.694 97.5605) (end 88.392 94.2585) (width 0.8) (layer "B.Cu") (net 8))
 (segment (start 93.726 102.108) (end 99.803949 96.030051) (width 0.8) (layer "B.Cu") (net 8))
 (segment (start 99.803949 90.405949) (end 102.851949 87.357949) (width 0.8) (layer "B.Cu") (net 8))
 (segment (start 86.614 90.424) (end 83.312 90.424) (width 0.8) (layer "B.Cu") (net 8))
 (segment (start 88.392 92.202) (end 86.614 90.424) (width 0.8) (layer "B.Cu") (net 8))
 (segment (start 105.290162 95.504) (end 104.430102 95.504) (width 0.8) (layer "B.Cu") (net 8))
 (segment (start 91.694 102.108) (end 93.726 102.108) (width 0.8) (layer "B.Cu") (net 8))
 (segment (start 88.392 94.2585) (end 88.392 92.202) (width 0.8) (layer "B.Cu") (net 8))
 (segment (start 99.803949 96.030051) (end 99.803949 90.405949) (width 0.8) (layer "B.Cu") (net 8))
 (segment (start 99.568 90.641898) (end 99.803949 90.405949) (width 0.8) (layer "B.Cu") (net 8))
 (segment (start 90.932 88.9) (end 82.55 88.9) (width 0.8) (layer "F.Cu") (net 2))
 (via (at 90.932 88.9) (size 1.8) (drill 1) (layers "F.Cu" "B.Cu") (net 2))
 (via (at 82.55 88.9) (size 1.8) (drill 1) (layers "F.Cu" "B.Cu") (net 2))
 (segment (start 88.854 85.09) (end 89.362 84.582) (width 0.8) (layer "B.Cu") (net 2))
 (segment (start 79.756 88.9) (end 82.55 88.9) (width 0.8) (layer "B.Cu") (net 2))
 (segment (start 89.362 84.582) (end 93.253 84.582) (width 0.8) (layer "B.Cu") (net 2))
 (segment (start 78.232 93.218) (end 78.232 90.424) (width 0.8) (layer "B.Cu") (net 2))
 (segment (start 78.232 90.424) (end 79.756 88.9) (width 0.8) (layer "B.Cu") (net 2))
 (segment (start 88.854 86.822) (end 88.854 85.09) (width 0.8) (layer "B.Cu") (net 2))
 (segment (start 90.932 88.9) (end 88.854 86.822) (width 0.8) (layer "B.Cu") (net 2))
 (segment (start 80.772 100.838) (end 80.772 103.632) (width 0.5) (layer "B.Cu") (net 3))
 (segment (start 45.512 90.932) (end 45.512 90.678) (width 0.8) (layer "B.Cu") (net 3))
 (segment (start 45.512 90.678) (end 45.512 84.79) (width 0.8) (layer "B.Cu") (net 3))
 (segment (start 36.345 99.845) (end 45.512 90.678) (width 0.5) (layer "B.Cu") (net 3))
 (segment (start 40.894 104.394) (end 36.345 99.845) (width 0.5) (layer "B.Cu") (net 3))
 (segment (start 55.326 91.44) (end 49.276 91.44) (width 0.8) (layer "B.Cu") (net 3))
 (segment (start 57.15 89.616) (end 55.326 91.44) (width 0.8) (layer "B.Cu") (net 3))
 (segment (start 46.02 91.44) (end 45.512 90.932) (width 0.8) (layer "B.Cu") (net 3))
 (segment (start 49.276 91.44) (end 46.02 91.44) (width 0.8) (layer "B.Cu") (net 3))
 (segment (start 80.01 104.394) (end 40.894 104.394) (width 0.5) (layer "B.Cu") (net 3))
 (segment (start 45.512 84.79) (end 45.72 84.582) (width 0.8) (layer "B.Cu") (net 3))
 (segment (start 80.772 103.632) (end 80.01 104.394) (width 0.5) (layer "B.Cu") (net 3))
 (segment (start 38.862 104.648) (end 38.227 104.013) (width 0.8) (layer "B.Cu") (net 7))
 (segment (start 33.333919 99.119919) (end 37.846 94.607838) (width 0.8) (layer "B.Cu") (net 7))
 (segment (start 85.852 100.838) (end 85.852 105.41) (width 0.5) (layer "B.Cu") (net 7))
 (segment (start 39.624 105.41) (end 38.227 104.013) (width 0.5) (layer "B.Cu") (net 7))
 (segment (start 37.846 94.607838) (end 37.846 90.17) (width 0.8) (layer "B.Cu") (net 7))
 (segment (start 37.846 90.17) (end 36.576 88.9) (width 0.8) (layer "B.Cu") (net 7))
 (segment (start 85.852 105.41) (end 39.624 105.41) (width 0.5) (layer "B.Cu") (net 7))
 (segment (start 38.227 104.013) (end 33.333919 99.119919) (width 0.8) (layer "B.Cu") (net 7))
 (segment (start 50.8 101.6) (end 50.038 100.838) (width 0.5) (layer "B.Cu") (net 10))
 (segment (start 60.118 90.758) (end 73.098 90.758) (width 0.5) (layer "B.Cu") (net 10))
 (segment (start 40.386 100.838) (end 39.116 99.568) (width 0.5) (layer "B.Cu") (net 10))
 (segment (start 73.098 90.758) (end 73.152 90.704) (width 0.5) (layer "B.Cu") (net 10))
 (segment (start 73.152 93.218) (end 73.152 90.704) (width 0.8) (layer "B.Cu") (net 10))
 (segment (start 50.038 100.838) (end 40.386 100.838) (width 0.5) (layer "B.Cu") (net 10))
 (segment (start 57.912 92.964) (end 60.118 90.758) (width 0.5) (layer "B.Cu") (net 10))
 (segment (start 39.116 99.568) (end 45.72 92.964) (width 0.5) (layer "B.Cu") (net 10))
 (segment (start 45.72 92.964) (end 57.912 92.964) (width 0.5) (layer "B.Cu") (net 10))
 (segment (start 53.34 101.6) (end 53.34 97.816) (width 0.5) (layer "B.Cu") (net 11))
 (segment (start 53.594 94.742) (end 53.594 97.562) (width 0.5) (layer "B.Cu") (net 11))
 (segment (start 68.326 93.218) (end 67.31 92.202) (width 0.5) (layer "B.Cu") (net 11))
 (segment (start 60.452 92.202) (end 57.912 94.742) (width 0.5) (layer "B.Cu") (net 11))
 (segment (start 67.31 92.202) (end 60.452 92.202) (width 0.5) (layer "B.Cu") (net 11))
 (segment (start 57.912 94.742) (end 53.594 94.742) (width 0.5) (layer "B.Cu") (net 11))
 (segment (start 53.594 97.562) (end 53.366 97.79) (width 0.5) (layer "B.Cu") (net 11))
 (segment (start 70.612 93.218) (end 68.326 93.218) (width 0.5) (layer "B.Cu") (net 11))
 (segment (start 53.34 97.816) (end 53.366 97.79) (width 0.5) (layer "B.Cu") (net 11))
 (segment (start 72.618 97.282) (end 72.618 97.764) (width 0.8) (layer "B.Cu") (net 5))
 (segment (start 73.152 98.298) (end 73.152 100.838) (width 0.8) (layer "B.Cu") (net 5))
 (segment (start 66.548 93.98) (end 60.452 93.98) (width 0.8) (layer "B.Cu") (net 5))
 (segment (start 60.452 93.98) (end 55.88 98.552) (width 0.8) (layer "B.Cu") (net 5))
 (segment (start 69.85 97.282) (end 66.548 93.98) (width 0.8) (layer "B.Cu") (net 5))
 (segment (start 55.88 98.552) (end 55.88 101.6) (width 0.8) (layer "B.Cu") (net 5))
 (segment (start 72.618 97.764) (end 73.152 98.298) (width 0.8) (layer "B.Cu") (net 5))
 (segment (start 72.618 97.282) (end 69.85 97.282) (width 0.8) (layer "B.Cu") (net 5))
 (segment (start 67.056 96.52) (end 67.056 99.288) (width 0.8) (layer "B.Cu") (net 4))
 (segment (start 69.088 99.314) (end 69.114 99.288) (width 0.8) (layer "B.Cu") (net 4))
 (segment (start 61.214 95.758) (end 66.294 95.758) (width 0.8) (layer "B.Cu") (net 4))
 (segment (start 69.088 99.314) (end 67.082 99.314) (width 0.8) (layer "B.Cu") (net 4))
 (segment (start 58.42 98.552) (end 61.214 95.758) (width 0.8) (layer "B.Cu") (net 4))
 (segment (start 58.42 101.6) (end 58.42 98.552) (width 0.8) (layer "B.Cu") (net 4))
 (segment (start 66.294 95.758) (end 67.056 96.52) (width 0.8) (layer "B.Cu") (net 4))
 (segment (start 70.612 100.838) (end 69.088 99.314) (width 0.8) (layer "B.Cu") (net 4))
 (segment (start 67.082 99.314) (end 67.056 99.288) (width 0.8) (layer "B.Cu") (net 4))
 (segment (start 80.772 95.758) (end 78.232 98.298) (width 0.8) (layer "B.Cu") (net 6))
 (segment (start 83.312 98.806) (end 88.392 98.806) (width 0.8) (layer "B.Cu") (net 6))
 (segment (start 83.312 100.838) (end 83.312 98.298) (width 0.8) (layer "B.Cu") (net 6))
 (segment (start 88.392 98.806) (end 89.916 100.33) (width 0.8) (layer "B.Cu") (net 6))
 (segment (start 85.852 95.758) (end 85.852 93.218) (width 0.8) (layer "B.Cu") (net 6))
 (segment (start 93.98 92.845) (end 93.228 92.093) (width 0.8) (layer "B.Cu") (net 6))
 (segment (start 83.312 98.298) (end 85.852 95.758) (width 0.8) (layer "B.Cu") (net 6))
 (segment (start 83.312 98.298) (end 80.772 95.758) (width 0.8) (layer "B.Cu") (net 6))
 (segment (start 80.772 95.758) (end 80.772 93.218) (width 0.8) (layer "B.Cu") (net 6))
 (segment (start 78.232 98.298) (end 78.232 100.838) (width 0.8) (layer "B.Cu") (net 6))
 (segment (start 89.916 100.33) (end 92.964 100.33) (width 0.8) (layer "B.Cu") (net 6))
 (segment (start 92.964 100.33) (end 93.98 99.314) (width 0.8) (layer "B.Cu") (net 6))
 (segment (start 93.98 99.314) (end 93.98 92.845) (width 0.8) (layer "B.Cu") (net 6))
 (segment (start 54.864 87.122) (end 64.262 87.122) (width 0.8) (layer "B.Cu") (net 12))
 (segment (start 65.024 86.36) (end 65.019 86.355) (width 0.8) (layer "B.Cu") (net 12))
 (segment (start 53.06 85.318) (end 54.864 87.122) (width 0.8) (layer "B.Cu") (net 12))
 (segment (start 52.832 85.318) (end 53.06 85.318) (width 0.8) (layer "B.Cu") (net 12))
 (segment (start 65.019 86.355) (end 65.019 84.582) (width 0.8) (layer "B.Cu") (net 12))
 (segment (start 64.262 87.122) (end 65.024 86.36) (width 0.8) (layer "B.Cu") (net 12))
 (segment (start 79.034 84.582) (end 82.082 81.534) (width 0.8) (layer "B.Cu") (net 14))
 (segment (start 82.082 81.534) (end 85.318 81.534) (width 0.8) (layer "B.Cu") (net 14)))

